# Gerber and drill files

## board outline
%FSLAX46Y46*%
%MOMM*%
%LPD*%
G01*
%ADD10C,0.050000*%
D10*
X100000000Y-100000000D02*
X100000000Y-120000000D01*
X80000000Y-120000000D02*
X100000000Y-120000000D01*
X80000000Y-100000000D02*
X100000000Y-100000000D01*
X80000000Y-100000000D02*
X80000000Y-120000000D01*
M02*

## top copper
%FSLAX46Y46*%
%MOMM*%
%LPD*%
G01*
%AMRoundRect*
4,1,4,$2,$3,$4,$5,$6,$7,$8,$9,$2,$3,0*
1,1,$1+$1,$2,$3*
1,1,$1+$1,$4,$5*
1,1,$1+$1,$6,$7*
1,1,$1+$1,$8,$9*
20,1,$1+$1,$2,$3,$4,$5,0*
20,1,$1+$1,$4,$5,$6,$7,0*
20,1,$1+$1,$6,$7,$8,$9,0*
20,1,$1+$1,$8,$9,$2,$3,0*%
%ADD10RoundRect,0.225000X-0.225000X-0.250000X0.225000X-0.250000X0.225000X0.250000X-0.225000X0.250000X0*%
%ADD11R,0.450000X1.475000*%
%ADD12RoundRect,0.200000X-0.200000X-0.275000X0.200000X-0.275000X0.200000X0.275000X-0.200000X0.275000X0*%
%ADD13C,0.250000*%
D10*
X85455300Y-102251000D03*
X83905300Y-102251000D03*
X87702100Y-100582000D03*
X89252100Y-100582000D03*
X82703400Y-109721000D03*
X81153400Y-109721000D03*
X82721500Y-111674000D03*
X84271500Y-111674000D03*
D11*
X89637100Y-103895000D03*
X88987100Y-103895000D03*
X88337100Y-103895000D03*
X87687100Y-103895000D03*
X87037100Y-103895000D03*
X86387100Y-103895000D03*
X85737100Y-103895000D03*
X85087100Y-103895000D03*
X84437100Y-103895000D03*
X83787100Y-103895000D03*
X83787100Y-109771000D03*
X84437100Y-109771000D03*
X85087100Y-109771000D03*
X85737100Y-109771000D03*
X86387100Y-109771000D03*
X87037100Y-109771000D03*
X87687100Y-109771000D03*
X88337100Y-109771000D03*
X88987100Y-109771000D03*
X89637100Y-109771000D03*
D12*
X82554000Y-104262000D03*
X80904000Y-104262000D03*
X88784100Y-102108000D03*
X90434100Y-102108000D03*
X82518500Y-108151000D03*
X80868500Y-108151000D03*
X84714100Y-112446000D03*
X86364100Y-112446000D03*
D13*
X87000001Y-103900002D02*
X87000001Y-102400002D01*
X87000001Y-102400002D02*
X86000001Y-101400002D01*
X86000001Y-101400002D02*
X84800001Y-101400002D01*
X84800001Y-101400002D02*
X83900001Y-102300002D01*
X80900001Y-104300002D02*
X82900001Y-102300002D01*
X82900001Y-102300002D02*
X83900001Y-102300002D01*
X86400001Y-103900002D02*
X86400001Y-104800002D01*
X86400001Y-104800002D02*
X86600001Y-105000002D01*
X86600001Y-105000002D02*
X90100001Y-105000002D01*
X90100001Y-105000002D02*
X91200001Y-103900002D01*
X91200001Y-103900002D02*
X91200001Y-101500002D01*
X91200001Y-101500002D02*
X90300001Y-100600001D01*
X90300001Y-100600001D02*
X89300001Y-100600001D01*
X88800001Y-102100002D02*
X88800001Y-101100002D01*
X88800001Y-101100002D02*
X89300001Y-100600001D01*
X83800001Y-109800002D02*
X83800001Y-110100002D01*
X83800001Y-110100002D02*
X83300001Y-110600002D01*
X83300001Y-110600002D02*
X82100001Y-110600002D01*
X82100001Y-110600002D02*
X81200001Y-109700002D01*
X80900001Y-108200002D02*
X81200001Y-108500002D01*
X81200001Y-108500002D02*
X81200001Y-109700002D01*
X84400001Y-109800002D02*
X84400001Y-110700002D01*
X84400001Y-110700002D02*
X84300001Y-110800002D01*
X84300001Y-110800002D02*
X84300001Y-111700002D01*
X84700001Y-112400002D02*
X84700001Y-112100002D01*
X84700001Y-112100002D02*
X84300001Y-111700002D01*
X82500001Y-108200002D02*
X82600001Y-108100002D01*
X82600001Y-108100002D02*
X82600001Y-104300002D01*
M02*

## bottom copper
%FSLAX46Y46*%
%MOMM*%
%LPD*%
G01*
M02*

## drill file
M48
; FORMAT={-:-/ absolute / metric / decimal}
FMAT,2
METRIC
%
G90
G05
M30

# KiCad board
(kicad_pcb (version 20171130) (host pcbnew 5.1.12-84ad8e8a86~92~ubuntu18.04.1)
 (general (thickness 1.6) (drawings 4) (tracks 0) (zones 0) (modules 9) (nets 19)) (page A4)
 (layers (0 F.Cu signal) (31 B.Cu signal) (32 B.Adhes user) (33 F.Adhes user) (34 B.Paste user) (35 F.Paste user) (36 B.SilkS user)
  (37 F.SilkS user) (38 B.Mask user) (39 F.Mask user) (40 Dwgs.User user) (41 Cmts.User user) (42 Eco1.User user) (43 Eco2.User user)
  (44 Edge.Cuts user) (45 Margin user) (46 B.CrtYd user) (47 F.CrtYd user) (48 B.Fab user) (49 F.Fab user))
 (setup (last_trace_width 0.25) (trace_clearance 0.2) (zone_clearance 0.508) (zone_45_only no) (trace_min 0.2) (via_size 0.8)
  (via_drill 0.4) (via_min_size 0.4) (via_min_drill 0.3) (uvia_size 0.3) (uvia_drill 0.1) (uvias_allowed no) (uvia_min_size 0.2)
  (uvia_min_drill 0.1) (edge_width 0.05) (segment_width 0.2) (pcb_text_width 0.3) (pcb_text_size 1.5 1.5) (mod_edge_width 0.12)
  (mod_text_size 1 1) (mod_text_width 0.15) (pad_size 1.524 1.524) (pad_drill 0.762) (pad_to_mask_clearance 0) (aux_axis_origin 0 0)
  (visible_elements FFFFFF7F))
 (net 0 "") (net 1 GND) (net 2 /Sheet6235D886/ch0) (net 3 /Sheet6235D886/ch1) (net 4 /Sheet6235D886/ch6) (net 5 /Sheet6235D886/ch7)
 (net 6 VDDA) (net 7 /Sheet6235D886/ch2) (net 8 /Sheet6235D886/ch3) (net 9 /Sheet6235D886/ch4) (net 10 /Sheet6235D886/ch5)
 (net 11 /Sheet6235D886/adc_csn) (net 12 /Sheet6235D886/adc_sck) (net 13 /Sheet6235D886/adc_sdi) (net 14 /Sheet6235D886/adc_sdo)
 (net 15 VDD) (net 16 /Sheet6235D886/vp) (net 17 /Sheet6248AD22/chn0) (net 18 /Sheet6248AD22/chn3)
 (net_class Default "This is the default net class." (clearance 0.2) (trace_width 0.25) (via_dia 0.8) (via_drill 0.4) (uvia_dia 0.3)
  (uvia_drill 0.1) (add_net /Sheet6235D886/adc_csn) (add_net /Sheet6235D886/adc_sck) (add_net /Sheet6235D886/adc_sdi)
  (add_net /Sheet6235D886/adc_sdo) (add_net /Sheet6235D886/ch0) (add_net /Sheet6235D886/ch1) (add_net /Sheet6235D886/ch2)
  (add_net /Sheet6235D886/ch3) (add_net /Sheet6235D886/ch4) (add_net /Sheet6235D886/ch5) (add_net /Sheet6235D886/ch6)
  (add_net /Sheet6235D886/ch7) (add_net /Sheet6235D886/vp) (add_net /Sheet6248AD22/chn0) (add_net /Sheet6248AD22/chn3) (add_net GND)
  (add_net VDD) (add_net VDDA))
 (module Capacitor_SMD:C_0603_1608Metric (layer F.Cu) (at 84.680300 102.251000)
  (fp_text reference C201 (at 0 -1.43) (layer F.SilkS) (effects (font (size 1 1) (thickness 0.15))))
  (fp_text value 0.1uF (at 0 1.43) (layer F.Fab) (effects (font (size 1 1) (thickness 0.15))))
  (pad 2 smd roundrect (at 0.775 0) (size 0.9 0.95) (layers F.Cu F.Mask F.Paste) (roundrect_rratio 0.25) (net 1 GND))
  (pad 1 smd roundrect (at -0.775 0) (size 0.9 0.95) (layers F.Cu F.Mask F.Paste) (roundrect_rratio 0.25) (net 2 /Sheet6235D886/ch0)))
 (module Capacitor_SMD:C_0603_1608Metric (layer F.Cu) (at 88.477100 100.582000)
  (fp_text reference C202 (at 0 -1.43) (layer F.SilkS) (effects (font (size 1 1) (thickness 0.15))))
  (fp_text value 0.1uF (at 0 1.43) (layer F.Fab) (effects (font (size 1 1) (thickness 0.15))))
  (pad 1 smd roundrect (at -0.775 0) (size 0.9 0.95) (layers F.Cu F.Mask F.Paste) (roundrect_rratio 0.25) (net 1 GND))
  (pad 2 smd roundrect (at 0.775 0) (size 0.9 0.95) (layers F.Cu F.Mask F.Paste) (roundrect_rratio 0.25) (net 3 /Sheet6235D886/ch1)))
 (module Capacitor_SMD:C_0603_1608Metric (layer F.Cu) (at 81.928400 109.721000)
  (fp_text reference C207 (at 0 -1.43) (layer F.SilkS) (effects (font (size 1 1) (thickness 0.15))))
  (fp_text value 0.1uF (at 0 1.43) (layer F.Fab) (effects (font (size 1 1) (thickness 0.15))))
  (pad 2 smd roundrect (at 0.775 0) (size 0.9 0.95) (layers F.Cu F.Mask F.Paste) (roundrect_rratio 0.25) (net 1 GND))
  (pad 1 smd roundrect (at -0.775 0) (size 0.9 0.95) (layers F.Cu F.Mask F.Paste) (roundrect_rratio 0.25) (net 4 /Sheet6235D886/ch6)))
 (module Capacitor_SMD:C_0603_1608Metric (layer F.Cu) (at 83.496500 111.674000)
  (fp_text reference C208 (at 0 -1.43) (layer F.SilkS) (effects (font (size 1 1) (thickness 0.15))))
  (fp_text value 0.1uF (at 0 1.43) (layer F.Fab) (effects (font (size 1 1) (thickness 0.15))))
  (pad 1 smd roundrect (at -0.775 0) (size 0.9 0.95) (layers F.Cu F.Mask F.Paste) (roundrect_rratio 0.25) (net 1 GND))
  (pad 2 smd roundrect (at 0.775 0) (size 0.9 0.95) (layers F.Cu F.Mask F.Paste) (roundrect_rratio 0.25) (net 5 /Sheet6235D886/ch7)))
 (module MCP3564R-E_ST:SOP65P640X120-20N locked (layer F.Cu) (at 86.712100 106.833000 270.000000)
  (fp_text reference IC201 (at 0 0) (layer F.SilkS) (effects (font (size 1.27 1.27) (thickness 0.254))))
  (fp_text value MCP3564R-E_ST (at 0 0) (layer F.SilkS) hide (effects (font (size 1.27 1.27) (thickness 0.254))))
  (pad 1 smd rect (at -2.938 -2.925) (size 0.45 1.475) (layers F.Cu F.Mask F.Paste) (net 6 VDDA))
  (pad 2 smd rect (at -2.938 -2.275) (size 0.45 1.475) (layers F.Cu F.Mask F.Paste) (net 1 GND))
  (pad 3 smd rect (at -2.938 -1.625) (size 0.45 1.475) (layers F.Cu F.Mask F.Paste) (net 1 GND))
  (pad 4 smd rect (at -2.938 -0.975) (size 0.45 1.475) (layers F.Cu F.Mask F.Paste))
  (pad 5 smd rect (at -2.938 -0.325) (size 0.45 1.475) (layers F.Cu F.Mask F.Paste) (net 2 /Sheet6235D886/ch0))
  (pad 6 smd rect (at -2.938 0.325) (size 0.45 1.475) (layers F.Cu F.Mask F.Paste) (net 3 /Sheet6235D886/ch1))
  (pad 7 smd rect (at -2.938 0.975) (size 0.45 1.475) (layers F.Cu F.Mask F.Paste) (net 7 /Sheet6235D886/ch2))
  (pad 8 smd rect (at -2.938 1.625) (size 0.45 1.475) (layers F.Cu F.Mask F.Paste) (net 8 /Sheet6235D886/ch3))
  (pad 9 smd rect (at -2.938 2.275) (size 0.45 1.475) (layers F.Cu F.Mask F.Paste) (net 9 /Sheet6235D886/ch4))
  (pad 10 smd rect (at -2.938 2.925) (size 0.45 1.475) (layers F.Cu F.Mask F.Paste) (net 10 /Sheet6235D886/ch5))
  (pad 11 smd rect (at 2.938 2.925) (size 0.45 1.475) (layers F.Cu F.Mask F.Paste) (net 4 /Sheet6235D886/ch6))
  (pad 12 smd rect (at 2.938 2.275) (size 0.45 1.475) (layers F.Cu F.Mask F.Paste) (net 5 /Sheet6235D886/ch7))
  (pad 13 smd rect (at 2.938 1.625) (size 0.45 1.475) (layers F.Cu F.Mask F.Paste) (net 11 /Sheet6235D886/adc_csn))
  (pad 14 smd rect (at 2.938 0.975) (size 0.45 1.475) (layers F.Cu F.Mask F.Paste) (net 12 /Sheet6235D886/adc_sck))
  (pad 15 smd rect (at 2.938 0.325) (size 0.45 1.475) (layers F.Cu F.Mask F.Paste) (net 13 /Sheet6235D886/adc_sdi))
  (pad 16 smd rect (at 2.938 -0.325) (size 0.45 1.475) (layers F.Cu F.Mask F.Paste) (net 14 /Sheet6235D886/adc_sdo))
  (pad 17 smd rect (at 2.938 -0.975) (size 0.45 1.475) (layers F.Cu F.Mask F.Paste))
  (pad 18 smd rect (at 2.938 -1.625) (size 0.45 1.475) (layers F.Cu F.Mask F.Paste))
  (pad 19 smd rect (at 2.938 -2.275) (size 0.45 1.475) (layers F.Cu F.Mask F.Paste) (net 1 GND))
  (pad 20 smd rect (at 2.938 -2.925) (size 0.45 1.475) (layers F.Cu F.Mask F.Paste) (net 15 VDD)))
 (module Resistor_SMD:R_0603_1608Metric (layer F.Cu) (at 81.729000 104.262000)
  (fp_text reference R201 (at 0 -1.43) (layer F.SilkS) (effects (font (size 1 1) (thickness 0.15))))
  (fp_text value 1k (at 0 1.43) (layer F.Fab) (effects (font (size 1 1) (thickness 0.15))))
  (pad 2 smd roundrect (at 0.825 0) (size 0.8 0.95) (layers F.Cu F.Mask F.Paste) (roundrect_rratio 0.25) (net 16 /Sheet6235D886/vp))
  (pad 1 smd roundrect (at -0.825 0) (size 0.8 0.95) (layers F.Cu F.Mask F.Paste) (roundrect_rratio 0.25) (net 2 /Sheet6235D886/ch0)))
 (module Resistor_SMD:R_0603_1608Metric (layer F.Cu) (at 89.609100 102.108000)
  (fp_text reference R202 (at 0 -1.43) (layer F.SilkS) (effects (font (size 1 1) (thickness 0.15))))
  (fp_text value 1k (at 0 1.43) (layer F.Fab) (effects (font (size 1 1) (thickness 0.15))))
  (pad 1 smd roundrect (at -0.825 0) (size 0.8 0.95) (layers F.Cu F.Mask F.Paste) (roundrect_rratio 0.25) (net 3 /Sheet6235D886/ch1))
  (pad 2 smd roundrect (at 0.825 0) (size 0.8 0.95) (layers F.Cu F.Mask F.Paste) (roundrect_rratio 0.25) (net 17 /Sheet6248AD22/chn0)))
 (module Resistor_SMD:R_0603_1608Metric (layer F.Cu) (at 81.693500 108.151000)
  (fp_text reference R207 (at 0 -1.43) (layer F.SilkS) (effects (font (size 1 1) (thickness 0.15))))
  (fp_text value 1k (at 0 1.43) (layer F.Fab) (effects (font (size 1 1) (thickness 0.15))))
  (pad 2 smd roundrect (at 0.825 0) (size 0.8 0.95) (layers F.Cu F.Mask F.Paste) (roundrect_rratio 0.25) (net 16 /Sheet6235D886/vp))
  (pad 1 smd roundrect (at -0.825 0) (size 0.8 0.95) (layers F.Cu F.Mask F.Paste) (roundrect_rratio 0.25) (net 4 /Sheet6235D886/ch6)))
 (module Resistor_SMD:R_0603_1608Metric (layer F.Cu) (at 85.539100 112.446000)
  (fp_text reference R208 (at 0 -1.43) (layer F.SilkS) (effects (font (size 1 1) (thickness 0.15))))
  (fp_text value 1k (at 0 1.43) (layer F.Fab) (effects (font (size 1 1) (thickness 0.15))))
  (pad 1 smd roundrect (at -0.825 0) (size 0.8 0.95) (layers F.Cu F.Mask F.Paste) (roundrect_rratio 0.25) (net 5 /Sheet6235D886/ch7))
  (pad 2 smd roundrect (at 0.825 0) (size 0.8 0.95) (layers F.Cu F.Mask F.Paste) (roundrect_rratio 0.25) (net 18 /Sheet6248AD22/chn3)))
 (gr_line (start 100 100) (end 100 120) (layer Edge.Cuts) (width 0.05))
 (gr_line (start 80 120) (end 100 120) (layer Edge.Cuts) (width 0.05))
 (gr_line (start 80 100) (end 100 100) (layer Edge.Cuts) (width 0.05))
 (gr_line (start 80 100) (end 80 120) (layer Edge.Cuts) (width 0.05))
 (segment (start 87.000001 103.900002) (end 87.000001 102.400002) (width 0.250000) (layer F.Cu) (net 2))
 (segment (start 87.000001 102.400002) (end 86.000001 101.400002) (width 0.250000) (layer F.Cu) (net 2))
 (segment (start 86.000001 101.400002) (end 84.800001 101.400002) (width 0.250000) (layer F.Cu) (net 2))
 (segment (start 84.800001 101.400002) (end 83.900001 102.300002) (width 0.250000) (layer F.Cu) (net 2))
 (segment (start 80.900001 104.300002) (end 82.900001 102.300002) (width 0.250000) (layer F.Cu) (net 2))
 (segment (start 82.900001 102.300002) (end 83.900001 102.300002) (width 0.250000) (layer F.Cu) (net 2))
 (segment (start 86.400001 103.900002) (end 86.400001 104.800002) (width 0.250000) (layer F.Cu) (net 3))
 (segment (start 86.400001 104.800002) (end 86.600001 105.000002) (width 0.250000) (layer F.Cu) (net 3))
 (segment (start 86.600001 105.000002) (end 90.100001 105.000002) (width 0.250000) (layer F.Cu) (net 3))
 (segment (start 90.100001 105.000002) (end 91.200001 103.900002) (width 0.250000) (layer F.Cu) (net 3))
 (segment (start 91.200001 103.900002) (end 91.200001 101.500002) (width 0.250000) (layer F.Cu) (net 3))
 (segment (start 91.200001 101.500002) (end 90.300001 100.600001) (width 0.250000) (layer F.Cu) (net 3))
 (segment (start 90.300001 100.600001) (end 89.300001 100.600001) (width 0.250000) (layer F.Cu) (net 3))
 (segment (start 88.800001 102.100002) (end 88.800001 101.100002) (width 0.250000) (layer F.Cu) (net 3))
 (segment (start 88.800001 101.100002) (end 89.300001 100.600001) (width 0.250000) (layer F.Cu) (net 3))
 (segment (start 83.800001 109.800002) (end 83.800001 110.100002) (width 0.250000) (layer F.Cu) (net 4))
 (segment (start 83.800001 110.100002) (end 83.300001 110.600002) (width 0.250000) (layer F.Cu) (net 4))
 (segment (start 83.300001 110.600002) (end 82.100001 110.600002) (width 0.250000) (layer F.Cu) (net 4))
 (segment (start 82.100001 110.600002) (end 81.200001 109.700002) (width 0.250000) (layer F.Cu) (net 4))
 (segment (start 80.900001 108.200002) (end 81.200001 108.500002) (width 0.250000) (layer F.Cu) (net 4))
 (segment (start 81.200001 108.500002) (end 81.200001 109.700002) (width 0.250000) (layer F.Cu) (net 4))
 (segment (start 84.400001 109.800002) (end 84.400001 110.700002) (width 0.250000) (layer F.Cu) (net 5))
 (segment (start 84.400001 110.700002) (end 84.300001 110.800002) (width 0.250000) (layer F.Cu) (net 5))
 (segment (start 84.300001 110.800002) (end 84.300001 111.700002) (width 0.250000) (layer F.Cu) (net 5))
 (segment (start 84.700001 112.400002) (end 84.700001 112.100002) (width 0.250000) (layer F.Cu) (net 5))
 (segment (start 84.700001 112.100002) (end 84.300001 111.700002) (width 0.250000) (layer F.Cu) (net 5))
 (segment (start 82.500001 108.200002) (end 82.600001 108.100002) (width 0.250000) (layer F.Cu) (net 16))
 (segment (start 82.600001 108.100002) (end 82.600001 104.300002) (width 0.250000) (layer F.Cu) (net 16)))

